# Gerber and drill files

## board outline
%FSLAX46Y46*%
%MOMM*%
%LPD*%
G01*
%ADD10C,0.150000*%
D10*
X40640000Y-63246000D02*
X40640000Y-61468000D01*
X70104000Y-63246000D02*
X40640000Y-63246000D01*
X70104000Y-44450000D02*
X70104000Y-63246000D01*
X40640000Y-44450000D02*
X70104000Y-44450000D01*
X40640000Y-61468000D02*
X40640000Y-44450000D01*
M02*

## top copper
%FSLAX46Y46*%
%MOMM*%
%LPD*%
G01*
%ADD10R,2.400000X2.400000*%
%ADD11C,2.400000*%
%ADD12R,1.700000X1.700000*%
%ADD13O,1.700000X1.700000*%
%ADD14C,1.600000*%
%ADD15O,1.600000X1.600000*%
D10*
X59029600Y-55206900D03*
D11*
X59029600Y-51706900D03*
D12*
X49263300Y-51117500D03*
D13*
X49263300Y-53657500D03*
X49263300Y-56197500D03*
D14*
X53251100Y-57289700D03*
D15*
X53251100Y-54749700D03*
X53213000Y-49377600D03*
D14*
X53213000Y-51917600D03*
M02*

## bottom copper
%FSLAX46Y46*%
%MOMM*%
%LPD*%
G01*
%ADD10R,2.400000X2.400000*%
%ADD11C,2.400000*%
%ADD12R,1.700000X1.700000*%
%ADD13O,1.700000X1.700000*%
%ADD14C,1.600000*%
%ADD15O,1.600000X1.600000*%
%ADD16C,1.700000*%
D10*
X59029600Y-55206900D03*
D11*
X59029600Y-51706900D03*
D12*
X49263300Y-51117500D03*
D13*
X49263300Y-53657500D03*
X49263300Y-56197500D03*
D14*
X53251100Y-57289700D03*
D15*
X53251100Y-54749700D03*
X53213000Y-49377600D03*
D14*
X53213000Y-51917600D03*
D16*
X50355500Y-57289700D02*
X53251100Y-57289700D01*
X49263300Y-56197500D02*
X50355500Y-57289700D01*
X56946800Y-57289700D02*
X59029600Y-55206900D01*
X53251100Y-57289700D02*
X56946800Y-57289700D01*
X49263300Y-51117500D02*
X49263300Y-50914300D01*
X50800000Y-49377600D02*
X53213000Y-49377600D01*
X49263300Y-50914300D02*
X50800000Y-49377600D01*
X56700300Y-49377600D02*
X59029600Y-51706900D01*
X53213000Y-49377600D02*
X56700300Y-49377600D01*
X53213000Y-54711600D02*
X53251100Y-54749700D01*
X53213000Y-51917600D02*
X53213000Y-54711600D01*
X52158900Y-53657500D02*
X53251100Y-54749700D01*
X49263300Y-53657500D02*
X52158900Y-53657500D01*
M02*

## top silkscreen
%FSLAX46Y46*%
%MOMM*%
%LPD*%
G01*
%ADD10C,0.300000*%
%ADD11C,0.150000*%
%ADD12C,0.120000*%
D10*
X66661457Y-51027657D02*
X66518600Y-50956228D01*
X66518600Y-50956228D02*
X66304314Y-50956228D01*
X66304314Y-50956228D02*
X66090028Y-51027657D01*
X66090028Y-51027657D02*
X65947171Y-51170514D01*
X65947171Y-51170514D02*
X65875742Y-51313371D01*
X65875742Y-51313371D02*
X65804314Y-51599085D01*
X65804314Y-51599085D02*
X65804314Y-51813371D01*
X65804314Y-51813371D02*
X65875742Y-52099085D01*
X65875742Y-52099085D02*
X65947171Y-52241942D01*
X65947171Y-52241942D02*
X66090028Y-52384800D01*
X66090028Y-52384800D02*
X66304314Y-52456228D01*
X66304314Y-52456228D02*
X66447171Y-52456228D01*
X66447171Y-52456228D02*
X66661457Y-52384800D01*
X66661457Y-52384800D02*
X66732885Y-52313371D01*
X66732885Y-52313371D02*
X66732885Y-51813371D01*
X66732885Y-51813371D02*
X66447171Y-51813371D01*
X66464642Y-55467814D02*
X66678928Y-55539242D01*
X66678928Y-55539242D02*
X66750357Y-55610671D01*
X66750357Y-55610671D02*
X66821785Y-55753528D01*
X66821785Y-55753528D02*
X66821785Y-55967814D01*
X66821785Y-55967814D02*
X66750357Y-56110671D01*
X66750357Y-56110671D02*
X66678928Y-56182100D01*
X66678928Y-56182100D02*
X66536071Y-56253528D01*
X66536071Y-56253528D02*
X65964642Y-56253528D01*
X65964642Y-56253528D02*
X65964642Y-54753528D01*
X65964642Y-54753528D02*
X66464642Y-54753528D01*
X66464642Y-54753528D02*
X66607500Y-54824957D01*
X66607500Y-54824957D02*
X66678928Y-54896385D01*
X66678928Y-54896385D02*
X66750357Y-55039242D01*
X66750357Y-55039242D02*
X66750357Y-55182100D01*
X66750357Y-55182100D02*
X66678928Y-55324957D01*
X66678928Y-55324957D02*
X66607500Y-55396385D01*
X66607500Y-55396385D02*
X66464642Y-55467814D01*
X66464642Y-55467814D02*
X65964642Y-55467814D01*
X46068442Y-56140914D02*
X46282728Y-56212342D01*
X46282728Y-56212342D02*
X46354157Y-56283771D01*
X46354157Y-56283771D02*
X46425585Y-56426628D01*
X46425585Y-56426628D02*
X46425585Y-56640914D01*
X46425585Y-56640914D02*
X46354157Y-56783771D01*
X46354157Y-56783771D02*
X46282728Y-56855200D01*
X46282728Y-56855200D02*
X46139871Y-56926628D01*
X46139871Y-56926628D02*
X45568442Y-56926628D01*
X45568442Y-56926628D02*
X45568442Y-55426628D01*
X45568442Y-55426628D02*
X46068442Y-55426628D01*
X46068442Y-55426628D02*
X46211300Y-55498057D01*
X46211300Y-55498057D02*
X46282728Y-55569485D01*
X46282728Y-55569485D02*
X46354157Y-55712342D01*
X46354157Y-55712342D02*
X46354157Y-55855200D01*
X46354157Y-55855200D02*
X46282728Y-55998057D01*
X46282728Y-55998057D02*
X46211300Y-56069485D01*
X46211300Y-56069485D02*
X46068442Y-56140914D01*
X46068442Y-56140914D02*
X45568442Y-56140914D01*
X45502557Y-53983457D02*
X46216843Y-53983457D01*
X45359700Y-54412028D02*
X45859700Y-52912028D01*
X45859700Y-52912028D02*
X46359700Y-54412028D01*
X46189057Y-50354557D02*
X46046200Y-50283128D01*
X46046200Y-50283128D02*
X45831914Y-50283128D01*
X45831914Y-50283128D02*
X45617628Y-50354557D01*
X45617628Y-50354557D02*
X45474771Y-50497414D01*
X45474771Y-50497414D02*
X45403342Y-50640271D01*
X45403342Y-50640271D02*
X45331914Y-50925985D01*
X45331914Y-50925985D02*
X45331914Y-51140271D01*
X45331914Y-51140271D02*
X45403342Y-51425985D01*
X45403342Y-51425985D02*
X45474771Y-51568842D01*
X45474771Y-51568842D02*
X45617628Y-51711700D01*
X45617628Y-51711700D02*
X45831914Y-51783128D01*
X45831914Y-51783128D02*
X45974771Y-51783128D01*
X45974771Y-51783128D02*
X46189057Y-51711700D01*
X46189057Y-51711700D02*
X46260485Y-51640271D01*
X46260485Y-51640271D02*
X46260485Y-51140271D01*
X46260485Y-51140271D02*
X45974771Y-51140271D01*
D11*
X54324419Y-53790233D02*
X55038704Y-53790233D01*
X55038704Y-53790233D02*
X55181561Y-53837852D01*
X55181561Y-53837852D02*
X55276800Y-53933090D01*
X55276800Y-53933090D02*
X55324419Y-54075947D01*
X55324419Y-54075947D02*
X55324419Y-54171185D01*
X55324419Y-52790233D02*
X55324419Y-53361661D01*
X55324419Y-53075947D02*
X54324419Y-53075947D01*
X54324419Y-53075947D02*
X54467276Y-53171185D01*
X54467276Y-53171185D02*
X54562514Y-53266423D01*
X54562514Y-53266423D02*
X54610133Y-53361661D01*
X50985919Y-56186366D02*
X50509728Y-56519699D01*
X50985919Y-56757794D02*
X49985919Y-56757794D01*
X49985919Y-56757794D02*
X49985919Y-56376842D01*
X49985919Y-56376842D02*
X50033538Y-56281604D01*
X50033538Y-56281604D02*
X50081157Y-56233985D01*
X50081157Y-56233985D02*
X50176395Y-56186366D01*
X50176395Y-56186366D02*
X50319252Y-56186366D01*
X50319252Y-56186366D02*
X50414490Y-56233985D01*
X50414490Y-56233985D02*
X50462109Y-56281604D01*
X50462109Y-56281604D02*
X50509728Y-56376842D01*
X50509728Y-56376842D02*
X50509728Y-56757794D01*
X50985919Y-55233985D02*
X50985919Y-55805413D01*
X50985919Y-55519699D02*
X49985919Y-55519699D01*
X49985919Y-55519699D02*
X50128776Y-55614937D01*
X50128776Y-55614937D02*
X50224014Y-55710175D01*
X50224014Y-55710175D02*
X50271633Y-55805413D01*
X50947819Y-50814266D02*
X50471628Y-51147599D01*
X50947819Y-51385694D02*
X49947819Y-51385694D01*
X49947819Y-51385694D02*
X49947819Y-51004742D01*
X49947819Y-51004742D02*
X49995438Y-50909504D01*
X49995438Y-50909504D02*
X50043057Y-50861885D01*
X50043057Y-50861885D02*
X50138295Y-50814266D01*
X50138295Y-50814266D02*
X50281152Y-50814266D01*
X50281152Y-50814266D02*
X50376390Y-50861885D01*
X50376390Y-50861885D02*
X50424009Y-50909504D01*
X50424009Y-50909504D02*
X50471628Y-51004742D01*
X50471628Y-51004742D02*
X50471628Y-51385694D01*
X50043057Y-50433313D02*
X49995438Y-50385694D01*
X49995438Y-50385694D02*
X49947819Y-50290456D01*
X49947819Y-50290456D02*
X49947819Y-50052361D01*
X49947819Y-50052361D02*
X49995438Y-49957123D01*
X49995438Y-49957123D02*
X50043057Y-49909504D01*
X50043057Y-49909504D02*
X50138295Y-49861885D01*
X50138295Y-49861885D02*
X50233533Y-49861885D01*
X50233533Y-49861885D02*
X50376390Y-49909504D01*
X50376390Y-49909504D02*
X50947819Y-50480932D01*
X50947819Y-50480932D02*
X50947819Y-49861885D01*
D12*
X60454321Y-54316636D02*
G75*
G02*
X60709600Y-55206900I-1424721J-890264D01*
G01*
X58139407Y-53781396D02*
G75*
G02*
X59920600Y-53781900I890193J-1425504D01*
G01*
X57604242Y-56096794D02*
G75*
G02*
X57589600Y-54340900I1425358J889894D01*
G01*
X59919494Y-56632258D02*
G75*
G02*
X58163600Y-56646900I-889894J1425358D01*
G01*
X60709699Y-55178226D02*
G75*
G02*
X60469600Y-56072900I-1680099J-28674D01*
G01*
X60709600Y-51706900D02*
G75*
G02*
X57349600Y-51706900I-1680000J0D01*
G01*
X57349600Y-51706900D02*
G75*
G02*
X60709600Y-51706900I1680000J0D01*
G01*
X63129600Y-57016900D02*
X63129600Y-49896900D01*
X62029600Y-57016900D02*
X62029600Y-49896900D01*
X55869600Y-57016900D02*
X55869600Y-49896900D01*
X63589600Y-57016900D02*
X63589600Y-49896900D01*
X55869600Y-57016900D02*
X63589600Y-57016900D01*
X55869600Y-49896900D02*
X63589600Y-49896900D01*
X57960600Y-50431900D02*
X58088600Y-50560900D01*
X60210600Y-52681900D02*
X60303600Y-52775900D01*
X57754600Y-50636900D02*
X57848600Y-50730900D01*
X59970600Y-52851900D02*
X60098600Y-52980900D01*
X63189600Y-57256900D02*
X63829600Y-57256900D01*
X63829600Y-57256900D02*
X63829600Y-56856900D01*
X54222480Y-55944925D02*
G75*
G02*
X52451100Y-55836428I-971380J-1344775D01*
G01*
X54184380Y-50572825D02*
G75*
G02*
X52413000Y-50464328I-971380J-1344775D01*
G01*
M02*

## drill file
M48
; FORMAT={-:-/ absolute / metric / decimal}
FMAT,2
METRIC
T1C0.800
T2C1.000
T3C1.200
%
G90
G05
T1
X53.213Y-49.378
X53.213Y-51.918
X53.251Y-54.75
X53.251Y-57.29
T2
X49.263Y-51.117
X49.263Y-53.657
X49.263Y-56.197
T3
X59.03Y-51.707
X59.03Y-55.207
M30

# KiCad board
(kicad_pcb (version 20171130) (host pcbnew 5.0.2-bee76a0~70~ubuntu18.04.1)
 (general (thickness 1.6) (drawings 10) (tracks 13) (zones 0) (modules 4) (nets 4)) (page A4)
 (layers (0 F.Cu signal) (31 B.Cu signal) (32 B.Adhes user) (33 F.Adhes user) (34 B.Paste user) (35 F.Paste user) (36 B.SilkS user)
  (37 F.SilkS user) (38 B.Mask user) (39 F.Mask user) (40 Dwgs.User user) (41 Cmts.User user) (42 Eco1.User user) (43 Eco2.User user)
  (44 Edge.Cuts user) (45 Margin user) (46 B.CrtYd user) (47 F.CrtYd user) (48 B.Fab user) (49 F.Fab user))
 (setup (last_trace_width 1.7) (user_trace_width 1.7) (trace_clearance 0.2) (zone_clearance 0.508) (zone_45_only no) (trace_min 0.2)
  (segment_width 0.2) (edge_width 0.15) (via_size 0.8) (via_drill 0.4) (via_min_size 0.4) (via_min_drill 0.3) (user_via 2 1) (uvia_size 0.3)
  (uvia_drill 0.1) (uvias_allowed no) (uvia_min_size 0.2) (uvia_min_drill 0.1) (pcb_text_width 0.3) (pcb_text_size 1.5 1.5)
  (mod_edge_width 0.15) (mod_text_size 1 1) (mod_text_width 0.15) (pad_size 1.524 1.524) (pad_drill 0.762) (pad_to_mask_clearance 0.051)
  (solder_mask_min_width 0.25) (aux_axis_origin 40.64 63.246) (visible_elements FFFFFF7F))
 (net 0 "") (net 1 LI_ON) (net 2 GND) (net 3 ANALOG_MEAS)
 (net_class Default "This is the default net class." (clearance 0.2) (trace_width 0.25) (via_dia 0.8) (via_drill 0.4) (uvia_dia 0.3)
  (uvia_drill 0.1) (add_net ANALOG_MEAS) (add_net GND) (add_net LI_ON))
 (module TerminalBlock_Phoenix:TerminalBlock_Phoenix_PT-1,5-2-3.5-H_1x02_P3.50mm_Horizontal (layer F.Cu) (at 59.0296 55.2069 90)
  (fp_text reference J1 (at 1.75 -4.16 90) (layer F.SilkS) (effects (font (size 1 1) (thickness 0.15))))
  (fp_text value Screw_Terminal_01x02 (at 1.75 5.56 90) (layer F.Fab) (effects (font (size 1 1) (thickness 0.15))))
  (fp_arc (start 0 0) (end 0 1.68) (angle -32) (layer F.SilkS) (width 0.12))
  (fp_arc (start 0 0) (end 1.425 0.891) (angle -64) (layer F.SilkS) (width 0.12))
  (fp_arc (start 0 0) (end 0.866 -1.44) (angle -63) (layer F.SilkS) (width 0.12))
  (fp_arc (start 0 0) (end -1.44 -0.866) (angle -63) (layer F.SilkS) (width 0.12))
  (fp_arc (start 0 0) (end -0.866 1.44) (angle -32) (layer F.SilkS) (width 0.12))
  (fp_circle (center 3.5 0) (end 5.18 0) (layer F.SilkS) (width 0.12))
  (fp_line (start -1.81 4.1) (end 5.31 4.1) (layer F.SilkS) (width 0.12))
  (fp_line (start -1.81 3) (end 5.31 3) (layer F.SilkS) (width 0.12))
  (fp_line (start -1.81 -3.16) (end 5.31 -3.16) (layer F.SilkS) (width 0.12))
  (fp_line (start -1.81 4.56) (end 5.31 4.56) (layer F.SilkS) (width 0.12))
  (fp_line (start -1.81 -3.16) (end -1.81 4.56) (layer F.SilkS) (width 0.12))
  (fp_line (start 5.31 -3.16) (end 5.31 4.56) (layer F.SilkS) (width 0.12))
  (fp_line (start 4.775 -1.069) (end 4.646 -0.941) (layer F.SilkS) (width 0.12))
  (fp_line (start 2.525 1.181) (end 2.431 1.274) (layer F.SilkS) (width 0.12))
  (fp_line (start 4.57 -1.275) (end 4.476 -1.181) (layer F.SilkS) (width 0.12))
  (fp_line (start 2.355 0.941) (end 2.226 1.069) (layer F.SilkS) (width 0.12))
  (fp_line (start -2.05 4.16) (end -2.05 4.8) (layer F.SilkS) (width 0.12))
  (fp_line (start -2.05 4.8) (end -1.65 4.8) (layer F.SilkS) (width 0.12))
  (pad 1 thru_hole rect (at 0 0 90) (size 2.4 2.4) (drill 1.2) (layers *.Cu *.Mask) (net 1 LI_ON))
  (pad 2 thru_hole circle (at 3.5 0 90) (size 2.4 2.4) (drill 1.2) (layers *.Cu *.Mask) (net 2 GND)))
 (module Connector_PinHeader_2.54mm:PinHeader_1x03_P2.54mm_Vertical (layer B.Cu) (at 49.2633 51.1175 180)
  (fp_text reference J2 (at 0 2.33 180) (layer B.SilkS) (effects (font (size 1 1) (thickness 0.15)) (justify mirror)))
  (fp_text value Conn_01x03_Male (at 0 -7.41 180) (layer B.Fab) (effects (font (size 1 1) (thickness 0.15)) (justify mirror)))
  (pad 1 thru_hole rect (at 0 0 180) (size 1.7 1.7) (drill 1) (layers *.Cu *.Mask) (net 2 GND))
  (pad 2 thru_hole oval (at 0 -2.54 180) (size 1.7 1.7) (drill 1) (layers *.Cu *.Mask) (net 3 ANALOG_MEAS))
  (pad 3 thru_hole oval (at 0 -5.08 180) (size 1.7 1.7) (drill 1) (layers *.Cu *.Mask) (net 1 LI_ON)))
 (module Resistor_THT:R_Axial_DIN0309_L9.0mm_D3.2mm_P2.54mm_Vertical (layer F.Cu) (at 53.2511 57.2897 90)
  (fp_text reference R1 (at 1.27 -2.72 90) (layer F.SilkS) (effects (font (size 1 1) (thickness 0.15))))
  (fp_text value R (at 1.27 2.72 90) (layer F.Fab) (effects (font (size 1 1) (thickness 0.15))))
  (fp_arc (start 0 0) (end 1.453272 -0.8) (angle -295.326041) (layer F.SilkS) (width 0.12))
  (pad 1 thru_hole circle (at 0 0 90) (size 1.6 1.6) (drill 0.8) (layers *.Cu *.Mask) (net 1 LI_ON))
  (pad 2 thru_hole oval (at 2.54 0 90) (size 1.6 1.6) (drill 0.8) (layers *.Cu *.Mask) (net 3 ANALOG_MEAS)))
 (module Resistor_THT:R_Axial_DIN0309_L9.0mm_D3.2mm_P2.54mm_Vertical (layer F.Cu) (at 53.213 51.9176 90)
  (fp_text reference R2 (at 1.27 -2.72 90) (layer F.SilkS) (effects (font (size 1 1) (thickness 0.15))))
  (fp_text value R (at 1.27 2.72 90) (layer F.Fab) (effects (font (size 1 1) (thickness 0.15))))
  (fp_arc (start 0 0) (end 1.453272 -0.8) (angle -295.326041) (layer F.SilkS) (width 0.12))
  (pad 2 thru_hole oval (at 2.54 0 90) (size 1.6 1.6) (drill 0.8) (layers *.Cu *.Mask) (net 2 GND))
  (pad 1 thru_hole circle (at 0 0 90) (size 1.6 1.6) (drill 0.8) (layers *.Cu *.Mask) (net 3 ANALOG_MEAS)))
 (gr_line (start 40.64 63.246) (end 40.64 61.468) (layer Edge.Cuts) (width 0.15))
 (gr_line (start 70.104 63.246) (end 40.64 63.246) (layer Edge.Cuts) (width 0.15))
 (gr_line (start 70.104 44.45) (end 70.104 63.246) (layer Edge.Cuts) (width 0.15))
 (gr_line (start 40.64 44.45) (end 70.104 44.45) (layer Edge.Cuts) (width 0.15))
 (gr_line (start 40.64 61.468) (end 40.64 44.45) (layer Edge.Cuts) (width 0.15))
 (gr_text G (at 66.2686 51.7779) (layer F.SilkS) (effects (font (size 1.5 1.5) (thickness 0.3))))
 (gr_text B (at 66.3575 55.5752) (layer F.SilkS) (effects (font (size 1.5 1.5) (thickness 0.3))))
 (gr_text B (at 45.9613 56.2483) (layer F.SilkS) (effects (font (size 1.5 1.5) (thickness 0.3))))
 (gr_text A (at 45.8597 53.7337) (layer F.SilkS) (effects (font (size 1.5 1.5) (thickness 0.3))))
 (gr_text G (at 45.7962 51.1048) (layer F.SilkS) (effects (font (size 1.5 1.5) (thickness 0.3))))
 (segment (start 50.3555 57.2897) (end 53.2511 57.2897) (width 1.7) (layer B.Cu) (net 1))
 (segment (start 49.2633 56.1975) (end 50.3555 57.2897) (width 1.7) (layer B.Cu) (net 1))
 (segment (start 56.9468 57.2897) (end 59.0296 55.2069) (width 1.7) (layer B.Cu) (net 1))
 (segment (start 53.2511 57.2897) (end 56.9468 57.2897) (width 1.7) (layer B.Cu) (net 1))
 (segment (start 49.2633 51.1175) (end 49.2633 50.9143) (width 1.7) (layer B.Cu) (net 2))
 (segment (start 50.8 49.3776) (end 53.213 49.3776) (width 1.7) (layer B.Cu) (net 2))
 (segment (start 49.2633 50.9143) (end 50.8 49.3776) (width 1.7) (layer B.Cu) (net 2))
 (segment (start 56.7003 49.3776) (end 59.0296 51.7069) (width 1.7) (layer B.Cu) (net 2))
 (segment (start 53.213 49.3776) (end 56.7003 49.3776) (width 1.7) (layer B.Cu) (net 2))
 (segment (start 53.213 54.7116) (end 53.2511 54.7497) (width 1.7) (layer B.Cu) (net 3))
 (segment (start 53.213 51.9176) (end 53.213 54.7116) (width 1.7) (layer B.Cu) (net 3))
 (segment (start 52.1589 53.6575) (end 53.2511 54.7497) (width 1.7) (layer B.Cu) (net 3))
 (segment (start 49.2633 53.6575) (end 52.1589 53.6575) (width 1.7) (layer B.Cu) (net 3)))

